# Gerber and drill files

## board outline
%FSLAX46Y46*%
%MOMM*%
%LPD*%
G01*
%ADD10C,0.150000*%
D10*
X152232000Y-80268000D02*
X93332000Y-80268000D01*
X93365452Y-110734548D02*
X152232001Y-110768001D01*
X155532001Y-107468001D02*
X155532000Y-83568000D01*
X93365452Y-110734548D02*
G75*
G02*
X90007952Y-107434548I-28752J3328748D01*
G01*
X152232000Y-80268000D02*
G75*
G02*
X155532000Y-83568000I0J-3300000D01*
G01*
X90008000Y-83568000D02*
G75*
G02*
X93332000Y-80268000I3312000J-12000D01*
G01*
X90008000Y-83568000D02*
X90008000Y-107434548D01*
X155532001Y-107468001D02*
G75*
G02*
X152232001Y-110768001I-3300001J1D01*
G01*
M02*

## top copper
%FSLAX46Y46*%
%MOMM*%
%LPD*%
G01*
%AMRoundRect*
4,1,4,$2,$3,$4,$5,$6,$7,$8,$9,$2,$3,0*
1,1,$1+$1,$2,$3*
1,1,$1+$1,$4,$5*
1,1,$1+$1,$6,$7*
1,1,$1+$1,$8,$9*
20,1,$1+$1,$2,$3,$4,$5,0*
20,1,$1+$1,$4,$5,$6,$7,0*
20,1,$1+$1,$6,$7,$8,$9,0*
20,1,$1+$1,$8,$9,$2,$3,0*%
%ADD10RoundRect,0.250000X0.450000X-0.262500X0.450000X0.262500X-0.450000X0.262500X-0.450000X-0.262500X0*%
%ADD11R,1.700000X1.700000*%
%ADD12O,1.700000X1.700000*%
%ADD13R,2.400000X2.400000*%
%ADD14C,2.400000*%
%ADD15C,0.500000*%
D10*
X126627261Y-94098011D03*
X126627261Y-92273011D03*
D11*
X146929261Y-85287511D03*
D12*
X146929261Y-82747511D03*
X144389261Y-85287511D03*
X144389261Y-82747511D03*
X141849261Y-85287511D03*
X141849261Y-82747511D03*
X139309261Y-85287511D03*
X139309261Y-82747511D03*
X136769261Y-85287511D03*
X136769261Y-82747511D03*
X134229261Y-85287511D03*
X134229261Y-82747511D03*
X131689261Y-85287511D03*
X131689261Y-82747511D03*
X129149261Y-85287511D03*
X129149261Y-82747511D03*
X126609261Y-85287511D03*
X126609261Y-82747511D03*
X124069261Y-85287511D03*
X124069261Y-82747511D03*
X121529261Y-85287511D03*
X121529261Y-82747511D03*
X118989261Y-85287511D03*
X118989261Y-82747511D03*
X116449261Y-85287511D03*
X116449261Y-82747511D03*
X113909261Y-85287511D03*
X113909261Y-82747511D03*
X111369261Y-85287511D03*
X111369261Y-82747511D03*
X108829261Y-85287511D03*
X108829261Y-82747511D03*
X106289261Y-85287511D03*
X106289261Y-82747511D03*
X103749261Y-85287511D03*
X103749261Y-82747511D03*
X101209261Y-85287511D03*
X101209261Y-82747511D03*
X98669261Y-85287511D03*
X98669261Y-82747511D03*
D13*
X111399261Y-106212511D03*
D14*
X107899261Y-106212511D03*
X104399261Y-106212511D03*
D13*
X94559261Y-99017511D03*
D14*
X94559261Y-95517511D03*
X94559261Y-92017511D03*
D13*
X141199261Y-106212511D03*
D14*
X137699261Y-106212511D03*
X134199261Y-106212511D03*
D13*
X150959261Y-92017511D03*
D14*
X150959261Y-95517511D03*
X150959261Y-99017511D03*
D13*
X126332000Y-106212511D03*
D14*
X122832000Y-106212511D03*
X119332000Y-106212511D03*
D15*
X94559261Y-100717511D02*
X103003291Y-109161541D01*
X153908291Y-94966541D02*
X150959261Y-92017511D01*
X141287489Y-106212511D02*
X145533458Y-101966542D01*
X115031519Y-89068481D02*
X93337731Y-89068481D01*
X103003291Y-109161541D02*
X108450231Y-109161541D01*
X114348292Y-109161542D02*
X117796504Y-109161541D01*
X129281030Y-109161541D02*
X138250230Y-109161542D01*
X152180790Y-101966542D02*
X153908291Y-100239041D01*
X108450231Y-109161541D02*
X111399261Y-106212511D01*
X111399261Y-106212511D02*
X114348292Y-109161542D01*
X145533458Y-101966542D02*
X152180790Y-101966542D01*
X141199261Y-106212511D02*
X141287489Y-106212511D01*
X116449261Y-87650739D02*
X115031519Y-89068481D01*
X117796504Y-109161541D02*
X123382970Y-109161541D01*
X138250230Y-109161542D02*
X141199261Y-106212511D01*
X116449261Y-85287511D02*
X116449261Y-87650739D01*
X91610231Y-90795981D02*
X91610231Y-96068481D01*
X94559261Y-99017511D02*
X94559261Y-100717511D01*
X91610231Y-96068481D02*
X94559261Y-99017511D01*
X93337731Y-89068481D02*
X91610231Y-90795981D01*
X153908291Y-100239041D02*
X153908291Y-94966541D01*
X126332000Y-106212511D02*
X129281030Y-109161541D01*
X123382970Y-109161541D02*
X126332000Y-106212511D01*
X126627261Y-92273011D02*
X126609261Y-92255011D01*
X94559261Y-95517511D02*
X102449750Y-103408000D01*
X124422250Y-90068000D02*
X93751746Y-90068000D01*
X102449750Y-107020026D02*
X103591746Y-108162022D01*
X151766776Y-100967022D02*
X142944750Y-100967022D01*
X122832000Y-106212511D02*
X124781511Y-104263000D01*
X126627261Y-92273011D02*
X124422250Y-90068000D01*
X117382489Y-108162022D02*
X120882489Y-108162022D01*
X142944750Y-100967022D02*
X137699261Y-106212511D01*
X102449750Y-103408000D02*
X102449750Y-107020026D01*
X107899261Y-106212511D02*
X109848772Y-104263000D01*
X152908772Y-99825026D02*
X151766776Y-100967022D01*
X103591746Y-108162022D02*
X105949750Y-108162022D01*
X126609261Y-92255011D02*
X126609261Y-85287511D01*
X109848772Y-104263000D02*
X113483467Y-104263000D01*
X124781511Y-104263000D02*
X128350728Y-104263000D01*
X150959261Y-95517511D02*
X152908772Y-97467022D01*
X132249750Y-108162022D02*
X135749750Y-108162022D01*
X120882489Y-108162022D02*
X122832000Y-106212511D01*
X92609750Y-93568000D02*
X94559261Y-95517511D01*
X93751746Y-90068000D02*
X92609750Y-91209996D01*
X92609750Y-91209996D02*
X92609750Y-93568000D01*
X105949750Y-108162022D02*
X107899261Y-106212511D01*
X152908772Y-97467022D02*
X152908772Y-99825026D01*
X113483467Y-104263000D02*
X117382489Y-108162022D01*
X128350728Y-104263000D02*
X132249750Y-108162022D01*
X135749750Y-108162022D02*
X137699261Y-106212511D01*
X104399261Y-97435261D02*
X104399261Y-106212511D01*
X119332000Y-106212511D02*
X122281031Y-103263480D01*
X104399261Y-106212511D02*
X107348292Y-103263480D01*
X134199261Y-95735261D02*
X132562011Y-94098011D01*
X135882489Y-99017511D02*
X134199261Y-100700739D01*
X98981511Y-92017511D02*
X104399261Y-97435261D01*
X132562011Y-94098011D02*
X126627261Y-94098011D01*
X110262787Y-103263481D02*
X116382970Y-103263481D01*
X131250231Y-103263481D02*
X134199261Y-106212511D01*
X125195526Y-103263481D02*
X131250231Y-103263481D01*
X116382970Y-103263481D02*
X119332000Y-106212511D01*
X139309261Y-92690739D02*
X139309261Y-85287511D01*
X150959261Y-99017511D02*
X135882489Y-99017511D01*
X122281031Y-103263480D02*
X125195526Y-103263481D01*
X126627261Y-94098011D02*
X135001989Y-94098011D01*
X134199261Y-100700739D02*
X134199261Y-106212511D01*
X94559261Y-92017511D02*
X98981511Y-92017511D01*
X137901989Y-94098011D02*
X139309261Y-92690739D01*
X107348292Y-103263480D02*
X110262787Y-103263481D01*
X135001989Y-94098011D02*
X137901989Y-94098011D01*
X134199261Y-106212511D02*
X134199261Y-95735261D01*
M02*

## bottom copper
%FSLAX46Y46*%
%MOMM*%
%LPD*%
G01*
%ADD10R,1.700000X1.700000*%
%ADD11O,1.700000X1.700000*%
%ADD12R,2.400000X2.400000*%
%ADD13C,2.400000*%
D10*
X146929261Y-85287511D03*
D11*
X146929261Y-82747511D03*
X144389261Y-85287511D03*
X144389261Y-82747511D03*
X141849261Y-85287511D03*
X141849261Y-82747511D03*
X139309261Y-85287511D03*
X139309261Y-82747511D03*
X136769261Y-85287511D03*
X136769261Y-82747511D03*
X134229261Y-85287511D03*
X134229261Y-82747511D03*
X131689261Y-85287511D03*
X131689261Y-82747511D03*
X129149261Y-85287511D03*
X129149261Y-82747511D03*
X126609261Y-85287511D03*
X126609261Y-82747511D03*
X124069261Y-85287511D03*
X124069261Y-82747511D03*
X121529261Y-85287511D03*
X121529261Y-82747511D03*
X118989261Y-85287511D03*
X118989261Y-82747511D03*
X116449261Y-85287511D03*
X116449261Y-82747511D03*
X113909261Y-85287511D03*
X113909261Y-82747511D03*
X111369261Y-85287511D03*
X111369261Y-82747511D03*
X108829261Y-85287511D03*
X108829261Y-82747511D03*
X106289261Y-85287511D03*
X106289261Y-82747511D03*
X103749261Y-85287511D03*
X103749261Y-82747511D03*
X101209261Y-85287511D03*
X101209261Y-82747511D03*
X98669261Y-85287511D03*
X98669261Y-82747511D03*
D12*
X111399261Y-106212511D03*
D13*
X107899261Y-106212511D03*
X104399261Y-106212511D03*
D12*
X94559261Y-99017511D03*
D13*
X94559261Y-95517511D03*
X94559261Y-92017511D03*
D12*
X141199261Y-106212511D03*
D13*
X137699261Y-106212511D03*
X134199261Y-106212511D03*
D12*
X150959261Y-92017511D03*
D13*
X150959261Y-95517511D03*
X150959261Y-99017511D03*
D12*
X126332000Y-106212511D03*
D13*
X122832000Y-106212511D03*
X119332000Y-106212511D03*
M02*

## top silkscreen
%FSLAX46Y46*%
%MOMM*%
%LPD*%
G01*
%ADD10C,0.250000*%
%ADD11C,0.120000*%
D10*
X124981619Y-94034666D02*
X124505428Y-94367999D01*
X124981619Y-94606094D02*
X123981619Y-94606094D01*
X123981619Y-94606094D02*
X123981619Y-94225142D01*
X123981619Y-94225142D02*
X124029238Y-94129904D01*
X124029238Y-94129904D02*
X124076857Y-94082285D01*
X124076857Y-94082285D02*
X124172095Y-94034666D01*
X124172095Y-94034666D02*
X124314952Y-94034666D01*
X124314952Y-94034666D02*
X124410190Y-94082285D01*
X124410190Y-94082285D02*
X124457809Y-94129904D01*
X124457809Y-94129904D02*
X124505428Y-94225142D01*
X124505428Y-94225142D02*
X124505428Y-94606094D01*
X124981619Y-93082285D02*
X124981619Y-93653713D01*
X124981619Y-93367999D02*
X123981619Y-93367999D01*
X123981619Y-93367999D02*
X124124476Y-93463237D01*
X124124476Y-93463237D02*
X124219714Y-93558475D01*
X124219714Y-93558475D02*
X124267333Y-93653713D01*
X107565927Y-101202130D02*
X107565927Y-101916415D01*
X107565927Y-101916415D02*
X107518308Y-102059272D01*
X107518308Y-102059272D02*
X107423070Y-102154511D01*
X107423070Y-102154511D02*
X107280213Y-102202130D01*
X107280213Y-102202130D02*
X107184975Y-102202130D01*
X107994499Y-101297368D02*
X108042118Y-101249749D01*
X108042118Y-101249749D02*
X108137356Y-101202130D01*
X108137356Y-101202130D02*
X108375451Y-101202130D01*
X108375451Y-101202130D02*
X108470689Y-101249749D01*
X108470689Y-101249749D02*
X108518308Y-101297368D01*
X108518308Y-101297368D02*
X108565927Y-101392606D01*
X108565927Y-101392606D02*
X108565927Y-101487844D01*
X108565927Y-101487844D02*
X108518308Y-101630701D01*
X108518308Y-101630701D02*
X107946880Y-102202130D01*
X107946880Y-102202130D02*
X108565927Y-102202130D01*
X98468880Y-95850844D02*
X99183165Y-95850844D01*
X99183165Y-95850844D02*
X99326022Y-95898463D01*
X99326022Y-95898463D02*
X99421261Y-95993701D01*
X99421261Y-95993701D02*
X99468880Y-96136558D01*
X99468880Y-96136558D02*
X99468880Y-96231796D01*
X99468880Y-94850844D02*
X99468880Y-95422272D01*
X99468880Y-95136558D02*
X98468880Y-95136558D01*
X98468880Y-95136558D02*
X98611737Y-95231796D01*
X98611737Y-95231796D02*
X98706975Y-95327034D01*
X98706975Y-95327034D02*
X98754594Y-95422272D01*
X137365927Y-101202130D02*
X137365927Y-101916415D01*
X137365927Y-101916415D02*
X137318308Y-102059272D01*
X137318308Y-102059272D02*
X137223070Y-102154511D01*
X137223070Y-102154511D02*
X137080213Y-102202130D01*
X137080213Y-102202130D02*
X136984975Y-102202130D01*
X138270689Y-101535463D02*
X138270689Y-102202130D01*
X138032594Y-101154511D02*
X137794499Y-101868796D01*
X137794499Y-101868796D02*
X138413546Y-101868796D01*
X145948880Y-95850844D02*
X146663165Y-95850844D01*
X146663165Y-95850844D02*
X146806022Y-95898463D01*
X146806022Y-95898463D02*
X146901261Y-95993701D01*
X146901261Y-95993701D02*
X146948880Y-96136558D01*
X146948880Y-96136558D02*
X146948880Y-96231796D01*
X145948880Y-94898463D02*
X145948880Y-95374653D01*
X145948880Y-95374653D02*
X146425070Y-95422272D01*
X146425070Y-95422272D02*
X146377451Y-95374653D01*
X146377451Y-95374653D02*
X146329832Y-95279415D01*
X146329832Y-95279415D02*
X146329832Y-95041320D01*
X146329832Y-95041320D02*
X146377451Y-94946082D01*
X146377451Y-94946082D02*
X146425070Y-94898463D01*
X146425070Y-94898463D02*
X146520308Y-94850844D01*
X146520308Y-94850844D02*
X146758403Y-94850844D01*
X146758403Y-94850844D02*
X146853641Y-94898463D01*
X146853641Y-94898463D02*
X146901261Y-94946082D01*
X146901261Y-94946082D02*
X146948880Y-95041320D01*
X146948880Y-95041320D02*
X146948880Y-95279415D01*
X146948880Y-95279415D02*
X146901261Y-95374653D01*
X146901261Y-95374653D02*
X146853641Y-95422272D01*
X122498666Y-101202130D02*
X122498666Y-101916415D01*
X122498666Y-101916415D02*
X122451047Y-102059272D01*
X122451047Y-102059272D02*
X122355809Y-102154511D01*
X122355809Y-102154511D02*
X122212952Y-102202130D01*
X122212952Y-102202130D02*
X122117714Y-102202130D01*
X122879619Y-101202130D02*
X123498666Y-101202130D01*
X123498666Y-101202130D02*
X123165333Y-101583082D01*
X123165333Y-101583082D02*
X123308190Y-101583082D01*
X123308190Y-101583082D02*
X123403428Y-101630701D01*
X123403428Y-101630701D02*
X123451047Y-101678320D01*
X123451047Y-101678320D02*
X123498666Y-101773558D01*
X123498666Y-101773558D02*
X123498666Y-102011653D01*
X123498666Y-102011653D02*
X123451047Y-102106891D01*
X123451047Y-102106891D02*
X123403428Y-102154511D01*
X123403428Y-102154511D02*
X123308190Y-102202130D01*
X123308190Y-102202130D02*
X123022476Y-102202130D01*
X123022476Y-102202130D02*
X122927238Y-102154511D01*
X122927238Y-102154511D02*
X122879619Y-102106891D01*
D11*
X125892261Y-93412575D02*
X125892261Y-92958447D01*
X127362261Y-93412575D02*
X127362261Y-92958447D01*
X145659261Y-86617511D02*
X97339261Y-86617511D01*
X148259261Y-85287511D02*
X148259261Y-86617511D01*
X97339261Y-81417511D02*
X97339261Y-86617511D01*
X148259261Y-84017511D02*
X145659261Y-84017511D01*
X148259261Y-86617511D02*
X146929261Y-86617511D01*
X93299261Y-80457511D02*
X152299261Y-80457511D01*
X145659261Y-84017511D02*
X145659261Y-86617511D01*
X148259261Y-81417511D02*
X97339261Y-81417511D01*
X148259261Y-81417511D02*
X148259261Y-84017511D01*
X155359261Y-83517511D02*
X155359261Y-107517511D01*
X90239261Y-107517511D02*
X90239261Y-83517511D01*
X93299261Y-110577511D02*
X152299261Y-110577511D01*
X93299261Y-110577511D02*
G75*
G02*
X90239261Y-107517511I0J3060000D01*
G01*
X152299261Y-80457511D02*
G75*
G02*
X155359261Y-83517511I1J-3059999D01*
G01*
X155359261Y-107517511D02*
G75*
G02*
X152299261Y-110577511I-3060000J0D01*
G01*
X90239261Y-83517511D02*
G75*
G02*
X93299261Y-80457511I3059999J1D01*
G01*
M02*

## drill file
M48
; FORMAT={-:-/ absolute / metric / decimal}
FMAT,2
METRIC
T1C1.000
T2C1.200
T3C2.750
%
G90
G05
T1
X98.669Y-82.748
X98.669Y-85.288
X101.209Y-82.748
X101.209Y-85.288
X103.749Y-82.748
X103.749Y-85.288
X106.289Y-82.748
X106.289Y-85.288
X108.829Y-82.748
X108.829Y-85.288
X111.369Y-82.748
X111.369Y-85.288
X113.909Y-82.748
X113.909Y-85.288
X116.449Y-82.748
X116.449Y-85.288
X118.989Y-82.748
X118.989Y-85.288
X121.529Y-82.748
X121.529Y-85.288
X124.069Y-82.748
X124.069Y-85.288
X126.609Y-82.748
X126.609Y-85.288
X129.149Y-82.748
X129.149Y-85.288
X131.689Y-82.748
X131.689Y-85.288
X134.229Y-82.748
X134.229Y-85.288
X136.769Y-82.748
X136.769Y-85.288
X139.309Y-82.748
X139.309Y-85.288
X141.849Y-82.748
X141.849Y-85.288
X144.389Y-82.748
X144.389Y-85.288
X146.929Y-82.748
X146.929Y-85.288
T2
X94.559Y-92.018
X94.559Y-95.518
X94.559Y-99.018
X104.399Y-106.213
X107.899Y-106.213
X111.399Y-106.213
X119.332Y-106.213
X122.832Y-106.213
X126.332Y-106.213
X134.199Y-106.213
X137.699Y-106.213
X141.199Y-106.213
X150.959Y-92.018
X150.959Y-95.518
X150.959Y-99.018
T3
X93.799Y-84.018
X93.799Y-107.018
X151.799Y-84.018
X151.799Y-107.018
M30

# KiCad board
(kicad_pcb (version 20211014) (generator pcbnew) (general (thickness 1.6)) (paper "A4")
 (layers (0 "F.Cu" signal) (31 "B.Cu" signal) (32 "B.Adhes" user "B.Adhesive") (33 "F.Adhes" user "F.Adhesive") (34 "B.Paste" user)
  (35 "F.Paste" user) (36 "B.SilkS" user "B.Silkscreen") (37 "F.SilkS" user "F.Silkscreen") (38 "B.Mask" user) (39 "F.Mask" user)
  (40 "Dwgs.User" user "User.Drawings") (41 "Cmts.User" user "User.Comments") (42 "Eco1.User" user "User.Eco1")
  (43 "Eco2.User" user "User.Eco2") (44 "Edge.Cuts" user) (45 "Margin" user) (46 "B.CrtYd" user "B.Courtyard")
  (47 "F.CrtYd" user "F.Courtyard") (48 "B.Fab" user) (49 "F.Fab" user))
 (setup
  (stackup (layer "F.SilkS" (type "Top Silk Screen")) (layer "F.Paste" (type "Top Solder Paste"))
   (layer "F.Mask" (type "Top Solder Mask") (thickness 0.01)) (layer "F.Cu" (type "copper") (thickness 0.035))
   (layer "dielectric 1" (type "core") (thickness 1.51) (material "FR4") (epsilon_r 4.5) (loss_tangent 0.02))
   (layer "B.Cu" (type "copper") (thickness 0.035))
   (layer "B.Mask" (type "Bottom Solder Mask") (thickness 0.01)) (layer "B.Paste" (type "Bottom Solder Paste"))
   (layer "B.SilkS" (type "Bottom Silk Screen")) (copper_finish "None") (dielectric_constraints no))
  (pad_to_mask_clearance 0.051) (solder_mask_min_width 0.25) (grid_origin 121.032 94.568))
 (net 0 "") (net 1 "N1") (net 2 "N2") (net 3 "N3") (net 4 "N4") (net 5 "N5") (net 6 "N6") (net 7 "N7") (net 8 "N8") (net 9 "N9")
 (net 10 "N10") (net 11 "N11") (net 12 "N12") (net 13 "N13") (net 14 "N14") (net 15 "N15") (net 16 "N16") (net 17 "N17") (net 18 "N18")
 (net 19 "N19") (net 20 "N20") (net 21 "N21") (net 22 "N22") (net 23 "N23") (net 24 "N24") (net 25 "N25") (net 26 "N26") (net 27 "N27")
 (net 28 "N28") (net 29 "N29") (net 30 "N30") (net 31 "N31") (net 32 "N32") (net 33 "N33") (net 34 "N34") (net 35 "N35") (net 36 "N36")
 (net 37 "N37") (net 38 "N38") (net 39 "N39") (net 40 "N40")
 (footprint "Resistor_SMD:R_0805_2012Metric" (layer "F.Cu") (at 126.627261 93.185511 90)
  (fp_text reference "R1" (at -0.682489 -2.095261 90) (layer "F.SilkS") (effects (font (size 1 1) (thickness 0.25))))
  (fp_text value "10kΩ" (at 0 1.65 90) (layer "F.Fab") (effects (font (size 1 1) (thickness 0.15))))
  (fp_line (start -0.227064 -0.735) (end 0.227064 -0.735) (layer "F.SilkS") (width 0.12))
  (fp_line (start -0.227064 0.735) (end 0.227064 0.735) (layer "F.SilkS") (width 0.12))
  (pad "1" smd roundrect (at -0.9125 0 90) (size 1.025 1.4) (layers "F.Cu" "F.Paste" "F.Mask") (roundrect_rratio 0.243902439) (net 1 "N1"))
  (pad "2" smd roundrect (at 0.9125 0 90) (size 1.025 1.4) (layers "F.Cu" "F.Paste" "F.Mask") (roundrect_rratio 0.243902439) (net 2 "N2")))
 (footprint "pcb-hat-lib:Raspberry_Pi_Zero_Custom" (layer "F.Cu") (at 146.929261 85.287511 -90)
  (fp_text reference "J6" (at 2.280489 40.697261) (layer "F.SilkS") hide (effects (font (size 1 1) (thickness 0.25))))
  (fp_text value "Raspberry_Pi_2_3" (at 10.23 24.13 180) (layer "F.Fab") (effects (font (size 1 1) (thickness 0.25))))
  (fp_line (start 1.33 1.27) (end 1.33 49.59) (layer "F.SilkS") (width 0.12))
  (fp_line (start 0 -1.33) (end 1.33 -1.33) (layer "F.SilkS") (width 0.12))
  (fp_line (start -3.87 49.59) (end 1.33 49.59) (layer "F.SilkS") (width 0.12))
  (fp_line (start -1.27 -1.33) (end -1.27 1.27) (layer "F.SilkS") (width 0.12))
  (fp_line (start 1.33 -1.33) (end 1.33 0) (layer "F.SilkS") (width 0.12))
  (fp_line (start -4.83 53.63) (end -4.83 -5.37) (layer "F.SilkS") (width 0.12))
  (fp_line (start -1.27 1.27) (end 1.33 1.27) (layer "F.SilkS") (width 0.12))
  (fp_line (start -3.87 -1.33) (end -3.87 49.59) (layer "F.SilkS") (width 0.12))
  (fp_line (start -3.87 -1.33) (end -1.27 -1.33) (layer "F.SilkS") (width 0.12))
  (fp_line (start -1.77 -8.43) (end 22.23 -8.43) (layer "F.SilkS") (width 0.12))
  (fp_line (start 22.23 56.69) (end -1.77 56.69) (layer "F.SilkS") (width 0.12))
  (fp_line (start 25.29 53.63) (end 25.29 -5.37) (layer "F.SilkS") (width 0.12))
  (fp_arc (start 25.29 53.63) (mid 24.393747 55.793747) (end 22.23 56.69) (layer "F.SilkS") (width 0.12))
  (fp_arc (start -4.83 -5.37) (mid -3.933747 -7.533747) (end -1.77 -8.43) (layer "F.SilkS") (width 0.12))
  (fp_arc (start 22.23 -8.43) (mid 24.393747 -7.533747) (end 25.29 -5.37) (layer "F.SilkS") (width 0.12))
  (fp_arc (start -1.77 56.69) (mid -3.933747 55.793747) (end -4.83 53.63) (layer "F.SilkS") (width 0.12))
  (pad "" np_thru_hole circle (at 21.73 53.13) (size 2.75 2.75) (drill 2.75) (layers *.Cu *.Mask) (solder_mask_margin 1.625))
  (pad "" np_thru_hole circle (at 21.73 -4.87) (size 2.75 2.75) (drill 2.75) (layers *.Cu *.Mask) (solder_mask_margin 1.625))
  (pad "" np_thru_hole circle (at -1.27 -4.87) (size 2.75 2.75) (drill 2.75) (layers *.Cu *.Mask) (solder_mask_margin 1.625))
  (pad "" np_thru_hole circle (at -1.27 53.13) (size 2.75 2.75) (drill 2.75) (layers *.Cu *.Mask) (solder_mask_margin 1.625))
  (pad "1" thru_hole rect (at 0 0 270) (size 1.7 1.7) (drill 1) (layers *.Cu *.Mask) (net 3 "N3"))
  (pad "2" thru_hole oval (at -2.54 0 270) (size 1.7 1.7) (drill 1) (layers *.Cu *.Mask) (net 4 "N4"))
  (pad "3" thru_hole oval (at 0 2.54 270) (size 1.7 1.7) (drill 1) (layers *.Cu *.Mask) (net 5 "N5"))
  (pad "4" thru_hole oval (at -2.54 2.54 270) (size 1.7 1.7) (drill 1) (layers *.Cu *.Mask) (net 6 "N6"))
  (pad "5" thru_hole oval (at 0 5.08 270) (size 1.7 1.7) (drill 1) (layers *.Cu *.Mask) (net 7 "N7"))
  (pad "6" thru_hole oval (at -2.54 5.08 270) (size 1.7 1.7) (drill 1) (layers *.Cu *.Mask) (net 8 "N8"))
  (pad "7" thru_hole oval (at 0 7.62 270) (size 1.7 1.7) (drill 1) (layers *.Cu *.Mask) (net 1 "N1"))
  (pad "8" thru_hole oval (at -2.54 7.62 270) (size 1.7 1.7) (drill 1) (layers *.Cu *.Mask) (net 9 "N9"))
  (pad "9" thru_hole oval (at 0 10.16 270) (size 1.7 1.7) (drill 1) (layers *.Cu *.Mask) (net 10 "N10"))
  (pad "10" thru_hole oval (at -2.54 10.16 270) (size 1.7 1.7) (drill 1) (layers *.Cu *.Mask) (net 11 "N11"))
  (pad "11" thru_hole oval (at 0 12.7 270) (size 1.7 1.7) (drill 1) (layers *.Cu *.Mask) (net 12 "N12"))
  (pad "12" thru_hole oval (at -2.54 12.7 270) (size 1.7 1.7) (drill 1) (layers *.Cu *.Mask) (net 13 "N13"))
  (pad "13" thru_hole oval (at 0 15.24 270) (size 1.7 1.7) (drill 1) (layers *.Cu *.Mask) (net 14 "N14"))
  (pad "14" thru_hole oval (at -2.54 15.24 270) (size 1.7 1.7) (drill 1) (layers *.Cu *.Mask) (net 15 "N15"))
  (pad "15" thru_hole oval (at 0 17.78 270) (size 1.7 1.7) (drill 1) (layers *.Cu *.Mask) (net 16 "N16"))
  (pad "16" thru_hole oval (at -2.54 17.78 270) (size 1.7 1.7) (drill 1) (layers *.Cu *.Mask) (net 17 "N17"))
  (pad "17" thru_hole oval (at 0 20.32 270) (size 1.7 1.7) (drill 1) (layers *.Cu *.Mask) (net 2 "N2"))
  (pad "18" thru_hole oval (at -2.54 20.32 270) (size 1.7 1.7) (drill 1) (layers *.Cu *.Mask) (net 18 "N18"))
  (pad "19" thru_hole oval (at 0 22.86 270) (size 1.7 1.7) (drill 1) (layers *.Cu *.Mask) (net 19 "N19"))
  (pad "20" thru_hole oval (at -2.54 22.86 270) (size 1.7 1.7) (drill 1) (layers *.Cu *.Mask) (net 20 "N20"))
  (pad "21" thru_hole oval (at 0 25.4 270) (size 1.7 1.7) (drill 1) (layers *.Cu *.Mask) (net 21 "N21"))
  (pad "22" thru_hole oval (at -2.54 25.4 270) (size 1.7 1.7) (drill 1) (layers *.Cu *.Mask) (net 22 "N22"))
  (pad "23" thru_hole oval (at 0 27.94 270) (size 1.7 1.7) (drill 1) (layers *.Cu *.Mask) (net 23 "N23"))
  (pad "24" thru_hole oval (at -2.54 27.94 270) (size 1.7 1.7) (drill 1) (layers *.Cu *.Mask) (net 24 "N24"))
  (pad "25" thru_hole oval (at 0 30.48 270) (size 1.7 1.7) (drill 1) (layers *.Cu *.Mask) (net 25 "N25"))
  (pad "26" thru_hole oval (at -2.54 30.48 270) (size 1.7 1.7) (drill 1) (layers *.Cu *.Mask) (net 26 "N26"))
  (pad "27" thru_hole oval (at 0 33.02 270) (size 1.7 1.7) (drill 1) (layers *.Cu *.Mask) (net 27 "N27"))
  (pad "28" thru_hole oval (at -2.54 33.02 270) (size 1.7 1.7) (drill 1) (layers *.Cu *.Mask) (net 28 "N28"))
  (pad "29" thru_hole oval (at 0 35.56 270) (size 1.7 1.7) (drill 1) (layers *.Cu *.Mask) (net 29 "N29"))
  (pad "30" thru_hole oval (at -2.54 35.56 270) (size 1.7 1.7) (drill 1) (layers *.Cu *.Mask) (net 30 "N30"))
  (pad "31" thru_hole oval (at 0 38.1 270) (size 1.7 1.7) (drill 1) (layers *.Cu *.Mask) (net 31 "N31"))
  (pad "32" thru_hole oval (at -2.54 38.1 270) (size 1.7 1.7) (drill 1) (layers *.Cu *.Mask) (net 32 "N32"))
  (pad "33" thru_hole oval (at 0 40.64 270) (size 1.7 1.7) (drill 1) (layers *.Cu *.Mask) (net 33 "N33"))
  (pad "34" thru_hole oval (at -2.54 40.64 270) (size 1.7 1.7) (drill 1) (layers *.Cu *.Mask) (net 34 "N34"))
  (pad "35" thru_hole oval (at 0 43.18 270) (size 1.7 1.7) (drill 1) (layers *.Cu *.Mask) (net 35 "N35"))
  (pad "36" thru_hole oval (at -2.54 43.18 270) (size 1.7 1.7) (drill 1) (layers *.Cu *.Mask) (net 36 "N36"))
  (pad "37" thru_hole oval (at 0 45.72 270) (size 1.7 1.7) (drill 1) (layers *.Cu *.Mask) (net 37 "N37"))
  (pad "38" thru_hole oval (at -2.54 45.72 270) (size 1.7 1.7) (drill 1) (layers *.Cu *.Mask) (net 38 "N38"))
  (pad "39" thru_hole oval (at 0 48.26 270) (size 1.7 1.7) (drill 1) (layers *.Cu *.Mask) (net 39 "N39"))
  (pad "40" thru_hole oval (at -2.54 48.26 270) (size 1.7 1.7) (drill 1) (layers *.Cu *.Mask) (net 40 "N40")))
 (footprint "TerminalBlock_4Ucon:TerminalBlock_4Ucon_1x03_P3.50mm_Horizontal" (layer "B.Cu") (at 111.399261 106.212511 180)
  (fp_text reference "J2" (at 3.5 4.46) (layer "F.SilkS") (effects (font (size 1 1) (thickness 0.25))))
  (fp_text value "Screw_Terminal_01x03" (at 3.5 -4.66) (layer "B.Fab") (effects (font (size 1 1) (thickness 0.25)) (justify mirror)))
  (pad "1" thru_hole rect (at 0 0 180) (size 2.4 2.4) (drill 1.2) (layers *.Cu *.Mask) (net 25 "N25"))
  (pad "2" thru_hole circle (at 3.5 0 180) (size 2.4 2.4) (drill 1.2) (layers *.Cu *.Mask) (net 2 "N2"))
  (pad "3" thru_hole circle (at 7 0 180) (size 2.4 2.4) (drill 1.2) (layers *.Cu *.Mask) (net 1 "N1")))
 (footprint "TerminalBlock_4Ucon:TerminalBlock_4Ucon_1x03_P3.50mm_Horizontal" (layer "B.Cu") (at 94.559261 99.017511 90)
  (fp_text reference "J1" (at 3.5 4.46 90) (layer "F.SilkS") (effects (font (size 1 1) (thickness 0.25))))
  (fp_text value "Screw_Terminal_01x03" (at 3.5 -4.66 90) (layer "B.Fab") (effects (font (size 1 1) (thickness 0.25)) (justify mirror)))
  (pad "1" thru_hole rect (at 0 0 90) (size 2.4 2.4) (drill 1.2) (layers *.Cu *.Mask) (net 25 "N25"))
  (pad "2" thru_hole circle (at 3.5 0 90) (size 2.4 2.4) (drill 1.2) (layers *.Cu *.Mask) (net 2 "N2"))
  (pad "3" thru_hole circle (at 7 0 90) (size 2.4 2.4) (drill 1.2) (layers *.Cu *.Mask) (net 1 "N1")))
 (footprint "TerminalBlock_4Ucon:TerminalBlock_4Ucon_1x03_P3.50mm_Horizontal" (layer "B.Cu") (at 141.199261 106.212511 180)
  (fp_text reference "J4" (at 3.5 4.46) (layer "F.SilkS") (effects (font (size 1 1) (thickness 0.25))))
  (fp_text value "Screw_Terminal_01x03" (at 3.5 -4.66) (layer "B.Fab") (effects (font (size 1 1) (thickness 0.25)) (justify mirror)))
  (pad "1" thru_hole rect (at 0 0 180) (size 2.4 2.4) (drill 1.2) (layers *.Cu *.Mask) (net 25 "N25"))
  (pad "2" thru_hole circle (at 3.5 0 180) (size 2.4 2.4) (drill 1.2) (layers *.Cu *.Mask) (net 2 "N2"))
  (pad "3" thru_hole circle (at 7 0 180) (size 2.4 2.4) (drill 1.2) (layers *.Cu *.Mask) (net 1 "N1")))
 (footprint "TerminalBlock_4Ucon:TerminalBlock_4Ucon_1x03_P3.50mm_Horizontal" (layer "B.Cu") (at 150.959261 92.017511 -90)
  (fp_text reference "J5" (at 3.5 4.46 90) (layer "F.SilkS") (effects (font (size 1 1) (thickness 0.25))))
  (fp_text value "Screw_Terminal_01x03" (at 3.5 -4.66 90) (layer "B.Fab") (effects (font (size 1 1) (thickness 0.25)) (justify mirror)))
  (pad "1" thru_hole rect (at 0 0 270) (size 2.4 2.4) (drill 1.2) (layers *.Cu *.Mask) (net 25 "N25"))
  (pad "2" thru_hole circle (at 3.5 0 270) (size 2.4 2.4) (drill 1.2) (layers *.Cu *.Mask) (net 2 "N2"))
  (pad "3" thru_hole circle (at 7 0 270) (size 2.4 2.4) (drill 1.2) (layers *.Cu *.Mask) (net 1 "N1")))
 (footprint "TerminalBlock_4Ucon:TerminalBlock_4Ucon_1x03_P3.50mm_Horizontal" (layer "B.Cu") (at 126.332 106.212511 180)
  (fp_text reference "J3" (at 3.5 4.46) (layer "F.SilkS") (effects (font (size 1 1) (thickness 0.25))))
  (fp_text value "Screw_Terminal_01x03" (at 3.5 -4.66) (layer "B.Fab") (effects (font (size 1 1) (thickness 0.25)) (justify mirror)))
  (pad "1" thru_hole rect (at 0 0 180) (size 2.4 2.4) (drill 1.2) (layers *.Cu *.Mask) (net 25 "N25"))
  (pad "2" thru_hole circle (at 3.5 0 180) (size 2.4 2.4) (drill 1.2) (layers *.Cu *.Mask) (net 2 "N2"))
  (pad "3" thru_hole circle (at 7 0 180) (size 2.4 2.4) (drill 1.2) (layers *.Cu *.Mask) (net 1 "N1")))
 (gr_line (start 152.232 80.268) (end 93.332 80.268) (layer "Edge.Cuts") (width 0.15))
 (gr_line (start 93.365452 110.734548) (end 152.232001 110.768001) (layer "Edge.Cuts") (width 0.15))
 (gr_line (start 155.532001 107.468001) (end 155.532 83.568) (layer "Edge.Cuts") (width 0.15))
 (gr_arc (start 93.365452 110.734548) (mid 91.003274 109.779899) (end 90.008 107.434548) (layer "Edge.Cuts") (width 0.15))
 (gr_arc (start 152.232 80.268) (mid 154.565452 81.234548) (end 155.532 83.568) (layer "Edge.Cuts") (width 0.15))
 (gr_arc (start 90.008 83.568) (mid 90.986548 81.229577) (end 93.332 80.268) (layer "Edge.Cuts") (width 0.15))
 (gr_line (start 90.008 83.568) (end 90.008 107.434548) (layer "Edge.Cuts") (width 0.15))
 (gr_arc (start 155.532001 107.468001) (mid 154.565453 109.801453) (end 152.232001 110.768001) (layer "Edge.Cuts") (width 0.15))
 (segment (start 94.559261 100.717511) (end 103.003291 109.161541) (width 0.5) (layer "F.Cu") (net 25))
 (segment (start 153.908291 94.966541) (end 150.959261 92.017511) (width 0.5) (layer "F.Cu") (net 25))
 (segment (start 141.287489 106.212511) (end 145.533458 101.966542) (width 0.5) (layer "F.Cu") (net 25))
 (segment (start 115.031519 89.068481) (end 93.337731 89.068481) (width 0.5) (layer "F.Cu") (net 25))
 (segment (start 103.003291 109.161541) (end 108.450231 109.161541) (width 0.5) (layer "F.Cu") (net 25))
 (segment (start 114.348292 109.161542) (end 117.796504 109.161541) (width 0.5) (layer "F.Cu") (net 25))
 (segment (start 129.28103 109.161541) (end 138.25023 109.161542) (width 0.5) (layer "F.Cu") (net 25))
 (segment (start 152.18079 101.966542) (end 153.908291 100.239041) (width 0.5) (layer "F.Cu") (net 25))
 (segment (start 108.450231 109.161541) (end 111.399261 106.212511) (width 0.5) (layer "F.Cu") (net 25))
 (segment (start 111.399261 106.212511) (end 114.348292 109.161542) (width 0.5) (layer "F.Cu") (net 25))
 (segment (start 145.533458 101.966542) (end 152.18079 101.966542) (width 0.5) (layer "F.Cu") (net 25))
 (segment (start 141.199261 106.212511) (end 141.287489 106.212511) (width 0.5) (layer "F.Cu") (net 25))
 (segment (start 116.449261 87.650739) (end 115.031519 89.068481) (width 0.5) (layer "F.Cu") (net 25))
 (segment (start 117.796504 109.161541) (end 123.38297 109.161541) (width 0.5) (layer "F.Cu") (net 25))
 (segment (start 138.25023 109.161542) (end 141.199261 106.212511) (width 0.5) (layer "F.Cu") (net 25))
 (segment (start 116.449261 85.287511) (end 116.449261 87.650739) (width 0.5) (layer "F.Cu") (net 25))
 (segment (start 91.610231 90.795981) (end 91.610231 96.068481) (width 0.5) (layer "F.Cu") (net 25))
 (segment (start 94.559261 99.017511) (end 94.559261 100.717511) (width 0.5) (layer "F.Cu") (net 25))
 (segment (start 91.610231 96.068481) (end 94.559261 99.017511) (width 0.5) (layer "F.Cu") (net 25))
 (segment (start 93.337731 89.068481) (end 91.610231 90.795981) (width 0.5) (layer "F.Cu") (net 25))
 (segment (start 153.908291 100.239041) (end 153.908291 94.966541) (width 0.5) (layer "F.Cu") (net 25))
 (segment (start 126.332 106.212511) (end 129.28103 109.161541) (width 0.5) (layer "F.Cu") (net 25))
 (segment (start 123.38297 109.161541) (end 126.332 106.212511) (width 0.5) (layer "F.Cu") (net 25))
 (segment (start 126.627261 92.273011) (end 126.609261 92.255011) (width 0.5) (layer "F.Cu") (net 2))
 (segment (start 94.559261 95.517511) (end 102.44975 103.408) (width 0.5) (layer "F.Cu") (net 2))
 (segment (start 124.42225 90.068) (end 93.751746 90.068) (width 0.5) (layer "F.Cu") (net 2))
 (segment (start 102.44975 107.020026) (end 103.591746 108.162022) (width 0.5) (layer "F.Cu") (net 2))
 (segment (start 151.766776 100.967022) (end 142.94475 100.967022) (width 0.5) (layer "F.Cu") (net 2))
 (segment (start 122.832 106.212511) (end 124.781511 104.263) (width 0.5) (layer "F.Cu") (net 2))
 (segment (start 126.627261 92.273011) (end 124.42225 90.068) (width 0.5) (layer "F.Cu") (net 2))
 (segment (start 117.382489 108.162022) (end 120.882489 108.162022) (width 0.5) (layer "F.Cu") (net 2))
 (segment (start 142.94475 100.967022) (end 137.699261 106.212511) (width 0.5) (layer "F.Cu") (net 2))
 (segment (start 102.44975 103.408) (end 102.44975 107.020026) (width 0.5) (layer "F.Cu") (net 2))
 (segment (start 107.899261 106.212511) (end 109.848772 104.263) (width 0.5) (layer "F.Cu") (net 2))
 (segment (start 152.908772 99.825026) (end 151.766776 100.967022) (width 0.5) (layer "F.Cu") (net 2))
 (segment (start 103.591746 108.162022) (end 105.94975 108.162022) (width 0.5) (layer "F.Cu") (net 2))
 (segment (start 126.609261 92.255011) (end 126.609261 85.287511) (width 0.5) (layer "F.Cu") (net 2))
 (segment (start 109.848772 104.263) (end 113.483467 104.263) (width 0.5) (layer "F.Cu") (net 2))
 (segment (start 124.781511 104.263) (end 128.350728 104.263) (width 0.5) (layer "F.Cu") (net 2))
 (segment (start 150.959261 95.517511) (end 152.908772 97.467022) (width 0.5) (layer "F.Cu") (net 2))
 (segment (start 132.24975 108.162022) (end 135.74975 108.162022) (width 0.5) (layer "F.Cu") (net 2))
 (segment (start 120.882489 108.162022) (end 122.832 106.212511) (width 0.5) (layer "F.Cu") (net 2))
 (segment (start 92.60975 93.568) (end 94.559261 95.517511) (width 0.5) (layer "F.Cu") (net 2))
 (segment (start 93.751746 90.068) (end 92.60975 91.209996) (width 0.5) (layer "F.Cu") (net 2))
 (segment (start 92.60975 91.209996) (end 92.60975 93.568) (width 0.5) (layer "F.Cu") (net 2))
 (segment (start 105.94975 108.162022) (end 107.899261 106.212511) (width 0.5) (layer "F.Cu") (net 2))
 (segment (start 152.908772 97.467022) (end 152.908772 99.825026) (width 0.5) (layer "F.Cu") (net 2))
 (segment (start 113.483467 104.263) (end 117.382489 108.162022) (width 0.5) (layer "F.Cu") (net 2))
 (segment (start 128.350728 104.263) (end 132.24975 108.162022) (width 0.5) (layer "F.Cu") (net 2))
 (segment (start 135.74975 108.162022) (end 137.699261 106.212511) (width 0.5) (layer "F.Cu") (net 2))
 (segment (start 104.399261 97.435261) (end 104.399261 106.212511) (width 0.5) (layer "F.Cu") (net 1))
 (segment (start 119.332 106.212511) (end 122.281031 103.26348) (width 0.5) (layer "F.Cu") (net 1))
 (segment (start 104.399261 106.212511) (end 107.348292 103.26348) (width 0.5) (layer "F.Cu") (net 1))
 (segment (start 134.199261 95.735261) (end 132.562011 94.098011) (width 0.5) (layer "F.Cu") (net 1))
 (segment (start 135.882489 99.017511) (end 134.199261 100.700739) (width 0.5) (layer "F.Cu") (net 1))
 (segment (start 98.981511 92.017511) (end 104.399261 97.435261) (width 0.5) (layer "F.Cu") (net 1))
 (segment (start 132.562011 94.098011) (end 126.627261 94.098011) (width 0.5) (layer "F.Cu") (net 1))
 (segment (start 110.262787 103.263481) (end 116.38297 103.263481) (width 0.5) (layer "F.Cu") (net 1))
 (segment (start 131.250231 103.263481) (end 134.199261 106.212511) (width 0.5) (layer "F.Cu") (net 1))
 (segment (start 125.195526 103.263481) (end 131.250231 103.263481) (width 0.5) (layer "F.Cu") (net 1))
 (segment (start 116.38297 103.263481) (end 119.332 106.212511) (width 0.5) (layer "F.Cu") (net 1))
 (segment (start 139.309261 92.690739) (end 139.309261 85.287511) (width 0.5) (layer "F.Cu") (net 1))
 (segment (start 150.959261 99.017511) (end 135.882489 99.017511) (width 0.5) (layer "F.Cu") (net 1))
 (segment (start 122.281031 103.26348) (end 125.195526 103.263481) (width 0.5) (layer "F.Cu") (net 1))
 (segment (start 126.627261 94.098011) (end 135.001989 94.098011) (width 0.5) (layer "F.Cu") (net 1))
 (segment (start 134.199261 100.700739) (end 134.199261 106.212511) (width 0.5) (layer "F.Cu") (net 1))
 (segment (start 94.559261 92.017511) (end 98.981511 92.017511) (width 0.5) (layer "F.Cu") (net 1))
 (segment (start 137.901989 94.098011) (end 139.309261 92.690739) (width 0.5) (layer "F.Cu") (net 1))
 (segment (start 107.348292 103.26348) (end 110.262787 103.263481) (width 0.5) (layer "F.Cu") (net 1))
 (segment (start 135.001989 94.098011) (end 137.901989 94.098011) (width 0.5) (layer "F.Cu") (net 1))
 (segment (start 134.199261 106.212511) (end 134.199261 95.735261) (width 0.5) (layer "F.Cu") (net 1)))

